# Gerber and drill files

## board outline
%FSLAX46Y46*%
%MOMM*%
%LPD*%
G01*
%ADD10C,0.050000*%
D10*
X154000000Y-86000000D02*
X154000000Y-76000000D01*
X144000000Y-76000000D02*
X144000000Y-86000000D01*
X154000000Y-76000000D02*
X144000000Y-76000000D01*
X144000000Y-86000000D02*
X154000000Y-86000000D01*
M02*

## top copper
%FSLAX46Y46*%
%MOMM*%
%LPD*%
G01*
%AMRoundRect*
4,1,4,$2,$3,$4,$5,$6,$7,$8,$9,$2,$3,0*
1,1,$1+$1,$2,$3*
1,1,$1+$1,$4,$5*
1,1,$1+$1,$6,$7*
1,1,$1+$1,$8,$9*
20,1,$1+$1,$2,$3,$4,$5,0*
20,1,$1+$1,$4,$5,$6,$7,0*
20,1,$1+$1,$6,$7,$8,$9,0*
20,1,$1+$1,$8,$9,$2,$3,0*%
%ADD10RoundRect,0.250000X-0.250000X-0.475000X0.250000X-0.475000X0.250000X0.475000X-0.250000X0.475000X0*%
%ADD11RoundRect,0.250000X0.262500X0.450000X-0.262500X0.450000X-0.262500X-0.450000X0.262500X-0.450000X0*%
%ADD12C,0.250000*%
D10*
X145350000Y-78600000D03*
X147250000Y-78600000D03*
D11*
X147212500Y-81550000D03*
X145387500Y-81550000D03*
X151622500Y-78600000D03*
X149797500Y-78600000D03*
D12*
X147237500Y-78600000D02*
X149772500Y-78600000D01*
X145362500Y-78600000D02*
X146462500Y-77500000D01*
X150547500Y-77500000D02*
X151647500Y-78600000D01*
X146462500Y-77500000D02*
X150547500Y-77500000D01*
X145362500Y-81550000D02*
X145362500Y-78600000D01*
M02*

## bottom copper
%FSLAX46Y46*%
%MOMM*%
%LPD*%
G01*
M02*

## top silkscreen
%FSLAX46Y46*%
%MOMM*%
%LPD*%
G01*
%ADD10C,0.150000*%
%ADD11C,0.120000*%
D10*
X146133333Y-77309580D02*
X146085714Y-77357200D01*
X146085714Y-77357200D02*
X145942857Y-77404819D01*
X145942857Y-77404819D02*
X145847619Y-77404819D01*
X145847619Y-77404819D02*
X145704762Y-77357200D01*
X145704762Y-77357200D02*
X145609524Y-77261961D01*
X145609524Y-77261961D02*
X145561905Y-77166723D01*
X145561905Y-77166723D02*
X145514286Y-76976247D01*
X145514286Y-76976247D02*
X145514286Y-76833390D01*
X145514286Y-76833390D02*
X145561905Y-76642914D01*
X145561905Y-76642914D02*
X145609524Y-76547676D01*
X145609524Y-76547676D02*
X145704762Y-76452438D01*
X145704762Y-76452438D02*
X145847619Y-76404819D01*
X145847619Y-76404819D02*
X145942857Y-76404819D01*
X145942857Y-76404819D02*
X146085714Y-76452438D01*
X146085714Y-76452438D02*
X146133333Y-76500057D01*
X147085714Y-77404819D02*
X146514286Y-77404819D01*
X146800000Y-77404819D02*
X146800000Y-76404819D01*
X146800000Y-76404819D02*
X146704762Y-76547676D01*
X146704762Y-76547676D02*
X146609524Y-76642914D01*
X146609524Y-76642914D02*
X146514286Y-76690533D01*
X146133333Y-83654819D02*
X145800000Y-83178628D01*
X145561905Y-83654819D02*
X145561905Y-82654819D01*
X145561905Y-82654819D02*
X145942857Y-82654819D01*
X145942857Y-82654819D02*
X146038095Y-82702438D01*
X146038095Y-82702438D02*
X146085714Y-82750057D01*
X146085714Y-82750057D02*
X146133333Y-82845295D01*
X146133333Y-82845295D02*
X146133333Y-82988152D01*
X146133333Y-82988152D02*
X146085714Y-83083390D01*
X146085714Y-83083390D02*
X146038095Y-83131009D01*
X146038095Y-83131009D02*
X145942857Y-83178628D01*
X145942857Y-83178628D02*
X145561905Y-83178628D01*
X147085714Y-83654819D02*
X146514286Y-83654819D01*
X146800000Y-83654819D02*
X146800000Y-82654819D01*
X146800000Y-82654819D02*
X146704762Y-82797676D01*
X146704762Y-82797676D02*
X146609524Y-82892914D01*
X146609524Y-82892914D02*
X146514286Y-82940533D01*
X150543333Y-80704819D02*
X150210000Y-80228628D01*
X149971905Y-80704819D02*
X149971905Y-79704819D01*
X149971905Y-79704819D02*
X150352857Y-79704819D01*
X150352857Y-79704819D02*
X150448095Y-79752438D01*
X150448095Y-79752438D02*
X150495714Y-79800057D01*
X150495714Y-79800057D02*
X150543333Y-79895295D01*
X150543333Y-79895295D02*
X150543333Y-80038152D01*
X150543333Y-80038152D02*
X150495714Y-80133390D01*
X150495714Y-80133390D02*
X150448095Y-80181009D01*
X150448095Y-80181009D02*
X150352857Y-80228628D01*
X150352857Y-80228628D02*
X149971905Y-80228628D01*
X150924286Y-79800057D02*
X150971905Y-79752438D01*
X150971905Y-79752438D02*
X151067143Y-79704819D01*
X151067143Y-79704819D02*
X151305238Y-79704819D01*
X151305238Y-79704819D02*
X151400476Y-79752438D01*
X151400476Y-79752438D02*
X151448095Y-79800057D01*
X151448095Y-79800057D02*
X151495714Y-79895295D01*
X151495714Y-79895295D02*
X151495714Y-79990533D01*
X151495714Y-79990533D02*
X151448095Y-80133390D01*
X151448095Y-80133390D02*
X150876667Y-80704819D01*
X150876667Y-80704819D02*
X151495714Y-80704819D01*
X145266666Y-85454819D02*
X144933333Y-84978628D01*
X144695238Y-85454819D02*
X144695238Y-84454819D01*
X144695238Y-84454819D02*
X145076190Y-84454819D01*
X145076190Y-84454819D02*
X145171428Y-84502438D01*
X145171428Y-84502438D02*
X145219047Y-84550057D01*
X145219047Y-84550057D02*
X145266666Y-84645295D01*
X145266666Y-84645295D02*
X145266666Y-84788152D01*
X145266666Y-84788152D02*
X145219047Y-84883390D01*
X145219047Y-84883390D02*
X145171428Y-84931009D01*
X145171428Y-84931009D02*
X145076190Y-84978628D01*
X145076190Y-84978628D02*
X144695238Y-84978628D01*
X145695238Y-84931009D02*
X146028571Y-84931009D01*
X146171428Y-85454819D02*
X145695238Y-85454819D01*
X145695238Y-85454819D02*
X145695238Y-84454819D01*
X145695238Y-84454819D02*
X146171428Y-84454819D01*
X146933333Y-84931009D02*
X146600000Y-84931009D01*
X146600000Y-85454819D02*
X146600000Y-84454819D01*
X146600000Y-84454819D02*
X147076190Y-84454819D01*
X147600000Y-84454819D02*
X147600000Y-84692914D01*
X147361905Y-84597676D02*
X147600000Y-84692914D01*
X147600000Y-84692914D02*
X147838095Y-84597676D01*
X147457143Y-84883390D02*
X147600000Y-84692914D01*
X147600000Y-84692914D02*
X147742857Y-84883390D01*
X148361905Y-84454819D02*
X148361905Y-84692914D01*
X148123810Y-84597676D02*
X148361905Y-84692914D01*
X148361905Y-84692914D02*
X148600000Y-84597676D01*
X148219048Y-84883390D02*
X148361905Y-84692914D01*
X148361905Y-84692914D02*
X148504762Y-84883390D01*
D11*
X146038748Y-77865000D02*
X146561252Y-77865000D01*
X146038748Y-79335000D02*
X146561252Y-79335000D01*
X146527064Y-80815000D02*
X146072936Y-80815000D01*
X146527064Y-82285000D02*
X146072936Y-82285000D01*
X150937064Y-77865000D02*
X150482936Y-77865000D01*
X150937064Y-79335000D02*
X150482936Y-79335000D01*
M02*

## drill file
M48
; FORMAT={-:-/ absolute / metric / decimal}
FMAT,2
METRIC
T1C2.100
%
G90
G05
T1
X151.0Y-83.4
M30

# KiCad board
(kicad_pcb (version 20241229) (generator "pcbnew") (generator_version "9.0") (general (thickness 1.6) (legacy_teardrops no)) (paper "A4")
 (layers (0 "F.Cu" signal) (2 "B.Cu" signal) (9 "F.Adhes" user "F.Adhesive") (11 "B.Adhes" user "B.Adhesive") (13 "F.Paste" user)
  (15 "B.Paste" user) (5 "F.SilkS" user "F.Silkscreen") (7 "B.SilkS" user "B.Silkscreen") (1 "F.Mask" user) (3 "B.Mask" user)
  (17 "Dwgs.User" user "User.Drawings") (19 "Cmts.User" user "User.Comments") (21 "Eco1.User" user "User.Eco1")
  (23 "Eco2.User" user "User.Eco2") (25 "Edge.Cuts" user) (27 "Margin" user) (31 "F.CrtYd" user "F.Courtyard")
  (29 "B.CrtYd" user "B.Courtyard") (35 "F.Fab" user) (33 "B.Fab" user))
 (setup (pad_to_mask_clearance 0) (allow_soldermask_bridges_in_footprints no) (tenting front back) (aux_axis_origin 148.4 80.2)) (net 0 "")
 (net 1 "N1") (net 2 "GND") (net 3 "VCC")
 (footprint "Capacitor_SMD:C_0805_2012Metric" (layer "F.Cu") (at 146.3 78.6)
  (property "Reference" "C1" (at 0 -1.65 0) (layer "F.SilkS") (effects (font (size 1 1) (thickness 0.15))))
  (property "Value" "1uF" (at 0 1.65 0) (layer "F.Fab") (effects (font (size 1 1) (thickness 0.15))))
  (fp_line (start -0.261252 -0.735) (end 0.261252 -0.735) (stroke (width 0.12) (type solid)) (layer "F.SilkS"))
  (fp_line (start -0.261252 0.735) (end 0.261252 0.735) (stroke (width 0.12) (type solid)) (layer "F.SilkS"))
  (pad "1" smd roundrect (at -0.95 0) (size 1 1.45) (layers "F.Cu" "F.Mask" "F.Paste") (roundrect_rratio 0.25) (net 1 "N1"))
  (pad "2" smd roundrect (at 0.95 0) (size 1 1.45) (layers "F.Cu" "F.Mask" "F.Paste") (roundrect_rratio 0.25) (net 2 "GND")))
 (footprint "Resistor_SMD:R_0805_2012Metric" (layer "F.Cu") (at 146.3 81.55 180)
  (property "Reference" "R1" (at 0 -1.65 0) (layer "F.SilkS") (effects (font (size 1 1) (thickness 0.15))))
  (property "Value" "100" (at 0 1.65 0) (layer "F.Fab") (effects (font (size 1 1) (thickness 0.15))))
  (fp_line (start -0.227064 0.735) (end 0.227064 0.735) (stroke (width 0.12) (type solid)) (layer "F.SilkS"))
  (fp_line (start -0.227064 -0.735) (end 0.227064 -0.735) (stroke (width 0.12) (type solid)) (layer "F.SilkS"))
  (pad "1" smd roundrect (at -0.9125 0 180) (size 1.025 1.4) (layers "F.Cu" "F.Mask" "F.Paste") (roundrect_rratio 0.243902) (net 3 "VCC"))
  (pad "2" smd roundrect (at 0.9125 0 180) (size 1.025 1.4) (layers "F.Cu" "F.Mask" "F.Paste") (roundrect_rratio 0.243902) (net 1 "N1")))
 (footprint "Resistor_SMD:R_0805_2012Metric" (layer "F.Cu") (at 150.71 78.6 180)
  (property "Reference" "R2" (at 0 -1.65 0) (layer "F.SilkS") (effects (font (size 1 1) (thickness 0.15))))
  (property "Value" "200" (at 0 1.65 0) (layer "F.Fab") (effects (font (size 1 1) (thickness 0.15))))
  (fp_line (start -0.227064 0.735) (end 0.227064 0.735) (stroke (width 0.12) (type solid)) (layer "F.SilkS"))
  (fp_line (start -0.227064 -0.735) (end 0.227064 -0.735) (stroke (width 0.12) (type solid)) (layer "F.SilkS"))
  (pad "1" smd roundrect (at -0.9125 0 180) (size 1.025 1.4) (layers "F.Cu" "F.Mask" "F.Paste") (roundrect_rratio 0.243902) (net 1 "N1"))
  (pad "2" smd roundrect (at 0.9125 0 180) (size 1.025 1.4) (layers "F.Cu" "F.Mask" "F.Paste") (roundrect_rratio 0.243902) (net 2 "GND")))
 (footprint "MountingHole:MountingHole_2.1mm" (layer "F.Cu") (at 151 83.4)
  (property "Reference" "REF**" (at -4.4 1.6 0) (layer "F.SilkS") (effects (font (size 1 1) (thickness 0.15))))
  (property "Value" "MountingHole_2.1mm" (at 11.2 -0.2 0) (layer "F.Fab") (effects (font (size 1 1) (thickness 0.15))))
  (pad "" np_thru_hole circle (at 0 0) (size 2.1 2.1) (drill 2.1) (layers "*.Cu" "*.Mask")))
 (gr_line (start 154 86) (end 154 76) (stroke (width 0.05) (type solid)) (layer "Edge.Cuts"))
 (gr_line (start 144 76) (end 144 86) (stroke (width 0.05) (type solid)) (layer "Edge.Cuts"))
 (gr_line (start 154 76) (end 144 76) (stroke (width 0.05) (type solid)) (layer "Edge.Cuts"))
 (gr_line (start 144 86) (end 154 86) (stroke (width 0.05) (type solid)) (layer "Edge.Cuts"))
 (segment (start 147.2375 78.6) (end 149.7725 78.6) (width 0.25) (layer "F.Cu") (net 2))
 (segment (start 145.3625 78.6) (end 146.4625 77.5) (width 0.25) (layer "F.Cu") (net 1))
 (segment (start 150.5475 77.5) (end 151.6475 78.6) (width 0.25) (layer "F.Cu") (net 1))
 (segment (start 146.4625 77.5) (end 150.5475 77.5) (width 0.25) (layer "F.Cu") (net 1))
 (segment (start 145.3625 81.55) (end 145.3625 78.6) (width 0.25) (layer "F.Cu") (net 1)))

